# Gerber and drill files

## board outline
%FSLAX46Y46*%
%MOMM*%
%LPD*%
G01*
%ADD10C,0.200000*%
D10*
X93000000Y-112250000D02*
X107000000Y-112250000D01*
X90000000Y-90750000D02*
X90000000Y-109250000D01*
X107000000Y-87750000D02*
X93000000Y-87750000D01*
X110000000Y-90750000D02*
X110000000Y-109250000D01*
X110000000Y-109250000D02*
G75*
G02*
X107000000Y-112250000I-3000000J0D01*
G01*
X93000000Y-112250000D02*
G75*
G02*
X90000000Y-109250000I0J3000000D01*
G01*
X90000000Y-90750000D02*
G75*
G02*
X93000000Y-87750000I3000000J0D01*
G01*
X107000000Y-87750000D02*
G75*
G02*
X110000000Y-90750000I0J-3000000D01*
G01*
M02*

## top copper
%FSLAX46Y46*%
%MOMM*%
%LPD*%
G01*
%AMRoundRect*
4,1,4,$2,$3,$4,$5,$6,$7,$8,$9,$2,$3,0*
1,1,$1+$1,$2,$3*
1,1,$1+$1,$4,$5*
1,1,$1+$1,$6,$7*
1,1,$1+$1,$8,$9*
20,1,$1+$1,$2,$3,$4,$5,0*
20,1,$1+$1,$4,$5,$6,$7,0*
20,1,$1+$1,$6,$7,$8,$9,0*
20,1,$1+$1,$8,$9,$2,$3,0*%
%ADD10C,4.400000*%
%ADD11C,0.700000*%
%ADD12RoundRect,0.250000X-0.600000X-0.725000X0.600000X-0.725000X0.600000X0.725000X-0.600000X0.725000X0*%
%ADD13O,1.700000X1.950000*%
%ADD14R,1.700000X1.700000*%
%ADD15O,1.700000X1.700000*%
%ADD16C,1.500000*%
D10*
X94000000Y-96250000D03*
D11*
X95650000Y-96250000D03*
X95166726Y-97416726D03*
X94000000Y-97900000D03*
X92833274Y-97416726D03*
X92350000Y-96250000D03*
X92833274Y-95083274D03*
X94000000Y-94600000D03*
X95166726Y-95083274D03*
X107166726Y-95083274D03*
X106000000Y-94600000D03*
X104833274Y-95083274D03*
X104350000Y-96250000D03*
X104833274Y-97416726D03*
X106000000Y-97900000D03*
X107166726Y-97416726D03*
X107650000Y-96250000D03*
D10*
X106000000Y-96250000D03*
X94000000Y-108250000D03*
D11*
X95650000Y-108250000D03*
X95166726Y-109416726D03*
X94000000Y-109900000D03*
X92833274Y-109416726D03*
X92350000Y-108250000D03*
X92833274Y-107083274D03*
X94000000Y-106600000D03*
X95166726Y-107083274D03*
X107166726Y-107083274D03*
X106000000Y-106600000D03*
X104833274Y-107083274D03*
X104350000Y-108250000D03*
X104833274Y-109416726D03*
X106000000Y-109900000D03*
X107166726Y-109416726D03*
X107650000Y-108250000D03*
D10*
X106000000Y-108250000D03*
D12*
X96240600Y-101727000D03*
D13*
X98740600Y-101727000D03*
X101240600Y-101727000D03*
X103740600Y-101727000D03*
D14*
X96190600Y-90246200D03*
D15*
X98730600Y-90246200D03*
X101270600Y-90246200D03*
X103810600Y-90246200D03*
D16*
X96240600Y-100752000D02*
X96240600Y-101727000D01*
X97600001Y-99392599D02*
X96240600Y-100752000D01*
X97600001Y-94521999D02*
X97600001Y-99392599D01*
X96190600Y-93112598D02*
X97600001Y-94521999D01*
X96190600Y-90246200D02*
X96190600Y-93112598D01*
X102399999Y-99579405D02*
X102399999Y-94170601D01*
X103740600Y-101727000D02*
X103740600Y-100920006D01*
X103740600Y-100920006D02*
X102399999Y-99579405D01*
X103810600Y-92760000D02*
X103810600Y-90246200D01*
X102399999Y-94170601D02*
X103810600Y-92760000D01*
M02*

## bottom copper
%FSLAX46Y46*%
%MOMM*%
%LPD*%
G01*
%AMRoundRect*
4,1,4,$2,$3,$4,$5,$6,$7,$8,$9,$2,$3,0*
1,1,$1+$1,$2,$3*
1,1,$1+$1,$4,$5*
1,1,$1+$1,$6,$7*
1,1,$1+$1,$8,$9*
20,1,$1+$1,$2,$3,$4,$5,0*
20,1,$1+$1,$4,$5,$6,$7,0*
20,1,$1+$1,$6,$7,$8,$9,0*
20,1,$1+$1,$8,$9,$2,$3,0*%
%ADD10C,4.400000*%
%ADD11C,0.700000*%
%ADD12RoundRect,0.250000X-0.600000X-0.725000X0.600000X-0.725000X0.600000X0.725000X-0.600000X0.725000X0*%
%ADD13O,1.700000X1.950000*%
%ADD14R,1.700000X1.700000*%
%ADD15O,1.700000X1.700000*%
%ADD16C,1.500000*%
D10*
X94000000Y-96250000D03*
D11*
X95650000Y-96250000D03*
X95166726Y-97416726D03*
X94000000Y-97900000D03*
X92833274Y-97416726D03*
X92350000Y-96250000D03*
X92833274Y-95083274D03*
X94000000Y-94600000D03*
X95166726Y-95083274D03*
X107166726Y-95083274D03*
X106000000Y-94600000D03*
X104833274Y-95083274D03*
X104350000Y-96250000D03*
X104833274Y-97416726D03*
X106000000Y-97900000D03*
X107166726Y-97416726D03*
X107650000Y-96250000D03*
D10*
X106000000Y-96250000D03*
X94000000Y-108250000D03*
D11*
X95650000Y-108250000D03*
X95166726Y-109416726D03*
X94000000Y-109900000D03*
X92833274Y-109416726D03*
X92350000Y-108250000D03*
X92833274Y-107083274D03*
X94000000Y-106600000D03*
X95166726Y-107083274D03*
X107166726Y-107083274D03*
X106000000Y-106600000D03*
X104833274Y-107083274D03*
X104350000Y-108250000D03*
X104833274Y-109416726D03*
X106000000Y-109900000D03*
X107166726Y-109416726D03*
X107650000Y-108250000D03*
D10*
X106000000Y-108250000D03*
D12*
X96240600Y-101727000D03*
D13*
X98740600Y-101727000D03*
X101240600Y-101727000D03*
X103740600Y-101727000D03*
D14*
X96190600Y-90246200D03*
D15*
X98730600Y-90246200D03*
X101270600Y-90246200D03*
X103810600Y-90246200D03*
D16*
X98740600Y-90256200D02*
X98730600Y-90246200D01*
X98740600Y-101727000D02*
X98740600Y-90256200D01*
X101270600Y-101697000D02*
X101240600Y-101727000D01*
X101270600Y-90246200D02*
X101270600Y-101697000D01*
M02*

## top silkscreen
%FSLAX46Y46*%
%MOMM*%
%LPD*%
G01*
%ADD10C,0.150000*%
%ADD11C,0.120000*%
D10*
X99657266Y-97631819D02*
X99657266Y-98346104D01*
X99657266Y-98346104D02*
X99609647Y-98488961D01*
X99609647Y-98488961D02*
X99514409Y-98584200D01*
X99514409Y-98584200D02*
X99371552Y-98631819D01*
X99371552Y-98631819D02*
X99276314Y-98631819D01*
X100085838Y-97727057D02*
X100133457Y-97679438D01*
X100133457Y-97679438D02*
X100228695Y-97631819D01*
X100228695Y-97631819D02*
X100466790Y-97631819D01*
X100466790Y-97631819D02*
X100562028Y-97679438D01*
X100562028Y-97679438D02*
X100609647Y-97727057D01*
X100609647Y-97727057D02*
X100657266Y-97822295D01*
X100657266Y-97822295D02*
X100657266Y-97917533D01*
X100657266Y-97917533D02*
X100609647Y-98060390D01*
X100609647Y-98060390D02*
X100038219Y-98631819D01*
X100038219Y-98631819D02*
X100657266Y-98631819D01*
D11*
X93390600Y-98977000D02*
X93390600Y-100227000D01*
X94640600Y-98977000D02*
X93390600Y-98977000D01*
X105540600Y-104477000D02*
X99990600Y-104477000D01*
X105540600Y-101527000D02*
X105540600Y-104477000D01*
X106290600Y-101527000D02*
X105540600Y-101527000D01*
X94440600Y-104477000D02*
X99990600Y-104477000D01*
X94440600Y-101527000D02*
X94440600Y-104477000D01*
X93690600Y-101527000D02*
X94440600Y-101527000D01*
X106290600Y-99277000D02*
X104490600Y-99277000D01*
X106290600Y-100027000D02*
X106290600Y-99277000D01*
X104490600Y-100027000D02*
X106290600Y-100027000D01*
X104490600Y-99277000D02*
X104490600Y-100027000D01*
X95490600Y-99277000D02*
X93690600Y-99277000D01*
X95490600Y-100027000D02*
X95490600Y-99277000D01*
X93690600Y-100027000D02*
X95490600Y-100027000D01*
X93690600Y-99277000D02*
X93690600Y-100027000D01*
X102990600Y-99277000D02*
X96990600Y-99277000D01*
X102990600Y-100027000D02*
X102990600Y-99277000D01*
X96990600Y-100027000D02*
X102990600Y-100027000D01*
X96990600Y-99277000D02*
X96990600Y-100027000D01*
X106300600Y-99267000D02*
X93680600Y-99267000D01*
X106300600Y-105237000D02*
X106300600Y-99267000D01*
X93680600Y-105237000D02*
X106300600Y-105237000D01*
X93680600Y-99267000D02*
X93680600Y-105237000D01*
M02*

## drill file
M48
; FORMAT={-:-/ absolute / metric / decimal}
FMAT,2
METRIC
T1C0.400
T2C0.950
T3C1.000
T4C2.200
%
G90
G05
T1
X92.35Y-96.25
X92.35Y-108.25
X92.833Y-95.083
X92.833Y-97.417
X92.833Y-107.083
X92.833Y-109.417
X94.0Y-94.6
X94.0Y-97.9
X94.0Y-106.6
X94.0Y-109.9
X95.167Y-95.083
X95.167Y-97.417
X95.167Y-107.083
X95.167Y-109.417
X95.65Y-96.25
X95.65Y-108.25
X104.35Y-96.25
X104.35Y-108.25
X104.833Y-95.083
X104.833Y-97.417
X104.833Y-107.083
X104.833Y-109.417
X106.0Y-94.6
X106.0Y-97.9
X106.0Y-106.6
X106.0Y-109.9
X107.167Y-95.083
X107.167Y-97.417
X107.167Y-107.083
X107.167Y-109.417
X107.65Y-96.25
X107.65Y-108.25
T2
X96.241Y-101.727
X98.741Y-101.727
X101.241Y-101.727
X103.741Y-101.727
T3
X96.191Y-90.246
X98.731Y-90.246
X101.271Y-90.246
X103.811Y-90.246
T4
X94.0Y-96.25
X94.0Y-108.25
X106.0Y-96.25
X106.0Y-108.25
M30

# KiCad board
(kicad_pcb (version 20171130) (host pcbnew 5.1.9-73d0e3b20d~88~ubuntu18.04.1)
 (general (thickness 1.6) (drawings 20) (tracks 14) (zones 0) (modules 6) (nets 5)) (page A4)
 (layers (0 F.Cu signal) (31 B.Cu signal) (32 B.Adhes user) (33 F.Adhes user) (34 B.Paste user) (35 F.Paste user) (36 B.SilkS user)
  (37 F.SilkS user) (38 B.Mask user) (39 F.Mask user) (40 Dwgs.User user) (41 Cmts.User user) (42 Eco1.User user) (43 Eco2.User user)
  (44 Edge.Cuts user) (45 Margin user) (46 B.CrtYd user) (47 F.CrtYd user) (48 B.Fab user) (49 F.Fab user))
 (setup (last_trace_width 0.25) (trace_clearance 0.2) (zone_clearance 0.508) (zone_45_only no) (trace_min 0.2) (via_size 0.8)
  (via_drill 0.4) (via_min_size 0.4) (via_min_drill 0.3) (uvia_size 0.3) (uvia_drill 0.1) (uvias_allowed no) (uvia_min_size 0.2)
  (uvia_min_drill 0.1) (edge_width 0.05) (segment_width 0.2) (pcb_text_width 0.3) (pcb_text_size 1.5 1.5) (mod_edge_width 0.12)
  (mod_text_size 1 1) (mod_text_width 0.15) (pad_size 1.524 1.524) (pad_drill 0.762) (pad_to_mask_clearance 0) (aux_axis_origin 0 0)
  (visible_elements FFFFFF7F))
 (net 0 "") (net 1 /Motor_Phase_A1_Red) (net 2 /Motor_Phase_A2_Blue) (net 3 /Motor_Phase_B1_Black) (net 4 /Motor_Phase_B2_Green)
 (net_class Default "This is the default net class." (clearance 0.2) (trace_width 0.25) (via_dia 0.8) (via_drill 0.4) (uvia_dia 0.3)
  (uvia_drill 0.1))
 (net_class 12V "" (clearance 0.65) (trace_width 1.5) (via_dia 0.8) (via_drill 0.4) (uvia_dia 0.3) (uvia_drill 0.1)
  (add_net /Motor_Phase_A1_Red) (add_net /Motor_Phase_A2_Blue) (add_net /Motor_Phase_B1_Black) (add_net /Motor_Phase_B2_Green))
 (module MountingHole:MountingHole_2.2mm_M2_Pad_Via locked (layer F.Cu) (at 94 96.25)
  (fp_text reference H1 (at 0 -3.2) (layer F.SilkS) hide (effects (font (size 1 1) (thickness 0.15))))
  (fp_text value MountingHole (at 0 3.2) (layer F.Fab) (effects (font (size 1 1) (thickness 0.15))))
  (pad 1 thru_hole circle (at 0 0) (size 4.4 4.4) (drill 2.2) (layers *.Cu *.Mask))
  (pad 1 thru_hole circle (at 1.65 0) (size 0.7 0.7) (drill 0.4) (layers *.Cu *.Mask))
  (pad 1 thru_hole circle (at 1.166726 1.166726) (size 0.7 0.7) (drill 0.4) (layers *.Cu *.Mask))
  (pad 1 thru_hole circle (at 0 1.65) (size 0.7 0.7) (drill 0.4) (layers *.Cu *.Mask))
  (pad 1 thru_hole circle (at -1.166726 1.166726) (size 0.7 0.7) (drill 0.4) (layers *.Cu *.Mask))
  (pad 1 thru_hole circle (at -1.65 0) (size 0.7 0.7) (drill 0.4) (layers *.Cu *.Mask))
  (pad 1 thru_hole circle (at -1.166726 -1.166726) (size 0.7 0.7) (drill 0.4) (layers *.Cu *.Mask))
  (pad 1 thru_hole circle (at 0 -1.65) (size 0.7 0.7) (drill 0.4) (layers *.Cu *.Mask))
  (pad 1 thru_hole circle (at 1.166726 -1.166726) (size 0.7 0.7) (drill 0.4) (layers *.Cu *.Mask)))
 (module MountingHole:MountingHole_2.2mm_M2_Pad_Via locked (layer F.Cu) (at 106 96.25)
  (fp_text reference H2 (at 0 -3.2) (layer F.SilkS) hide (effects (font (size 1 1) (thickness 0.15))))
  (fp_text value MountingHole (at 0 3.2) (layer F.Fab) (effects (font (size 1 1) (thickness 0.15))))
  (pad 1 thru_hole circle (at 1.166726 -1.166726) (size 0.7 0.7) (drill 0.4) (layers *.Cu *.Mask))
  (pad 1 thru_hole circle (at 0 -1.65) (size 0.7 0.7) (drill 0.4) (layers *.Cu *.Mask))
  (pad 1 thru_hole circle (at -1.166726 -1.166726) (size 0.7 0.7) (drill 0.4) (layers *.Cu *.Mask))
  (pad 1 thru_hole circle (at -1.65 0) (size 0.7 0.7) (drill 0.4) (layers *.Cu *.Mask))
  (pad 1 thru_hole circle (at -1.166726 1.166726) (size 0.7 0.7) (drill 0.4) (layers *.Cu *.Mask))
  (pad 1 thru_hole circle (at 0 1.65) (size 0.7 0.7) (drill 0.4) (layers *.Cu *.Mask))
  (pad 1 thru_hole circle (at 1.166726 1.166726) (size 0.7 0.7) (drill 0.4) (layers *.Cu *.Mask))
  (pad 1 thru_hole circle (at 1.65 0) (size 0.7 0.7) (drill 0.4) (layers *.Cu *.Mask))
  (pad 1 thru_hole circle (at 0 0) (size 4.4 4.4) (drill 2.2) (layers *.Cu *.Mask)))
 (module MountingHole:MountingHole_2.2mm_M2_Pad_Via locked (layer F.Cu) (at 94 108.25)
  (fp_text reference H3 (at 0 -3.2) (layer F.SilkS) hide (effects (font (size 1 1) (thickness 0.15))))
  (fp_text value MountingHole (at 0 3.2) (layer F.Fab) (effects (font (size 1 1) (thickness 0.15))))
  (pad 1 thru_hole circle (at 0 0) (size 4.4 4.4) (drill 2.2) (layers *.Cu *.Mask))
  (pad 1 thru_hole circle (at 1.65 0) (size 0.7 0.7) (drill 0.4) (layers *.Cu *.Mask))
  (pad 1 thru_hole circle (at 1.166726 1.166726) (size 0.7 0.7) (drill 0.4) (layers *.Cu *.Mask))
  (pad 1 thru_hole circle (at 0 1.65) (size 0.7 0.7) (drill 0.4) (layers *.Cu *.Mask))
  (pad 1 thru_hole circle (at -1.166726 1.166726) (size 0.7 0.7) (drill 0.4) (layers *.Cu *.Mask))
  (pad 1 thru_hole circle (at -1.65 0) (size 0.7 0.7) (drill 0.4) (layers *.Cu *.Mask))
  (pad 1 thru_hole circle (at -1.166726 -1.166726) (size 0.7 0.7) (drill 0.4) (layers *.Cu *.Mask))
  (pad 1 thru_hole circle (at 0 -1.65) (size 0.7 0.7) (drill 0.4) (layers *.Cu *.Mask))
  (pad 1 thru_hole circle (at 1.166726 -1.166726) (size 0.7 0.7) (drill 0.4) (layers *.Cu *.Mask)))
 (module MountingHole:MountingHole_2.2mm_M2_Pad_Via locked (layer F.Cu) (at 106 108.25)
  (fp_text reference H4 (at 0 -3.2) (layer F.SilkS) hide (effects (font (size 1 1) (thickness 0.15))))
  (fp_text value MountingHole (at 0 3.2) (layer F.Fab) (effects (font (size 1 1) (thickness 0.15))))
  (pad 1 thru_hole circle (at 1.166726 -1.166726) (size 0.7 0.7) (drill 0.4) (layers *.Cu *.Mask))
  (pad 1 thru_hole circle (at 0 -1.65) (size 0.7 0.7) (drill 0.4) (layers *.Cu *.Mask))
  (pad 1 thru_hole circle (at -1.166726 -1.166726) (size 0.7 0.7) (drill 0.4) (layers *.Cu *.Mask))
  (pad 1 thru_hole circle (at -1.65 0) (size 0.7 0.7) (drill 0.4) (layers *.Cu *.Mask))
  (pad 1 thru_hole circle (at -1.166726 1.166726) (size 0.7 0.7) (drill 0.4) (layers *.Cu *.Mask))
  (pad 1 thru_hole circle (at 0 1.65) (size 0.7 0.7) (drill 0.4) (layers *.Cu *.Mask))
  (pad 1 thru_hole circle (at 1.166726 1.166726) (size 0.7 0.7) (drill 0.4) (layers *.Cu *.Mask))
  (pad 1 thru_hole circle (at 1.65 0) (size 0.7 0.7) (drill 0.4) (layers *.Cu *.Mask))
  (pad 1 thru_hole circle (at 0 0) (size 4.4 4.4) (drill 2.2) (layers *.Cu *.Mask)))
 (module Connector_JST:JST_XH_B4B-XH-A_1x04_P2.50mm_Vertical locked (layer F.Cu) (at 96.2406 101.727)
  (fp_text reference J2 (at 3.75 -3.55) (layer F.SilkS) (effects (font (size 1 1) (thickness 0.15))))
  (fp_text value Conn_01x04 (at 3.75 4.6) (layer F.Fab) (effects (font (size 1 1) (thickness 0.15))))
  (fp_line (start -2.85 -2.75) (end -2.85 -1.5) (layer F.SilkS) (width 0.12))
  (fp_line (start -1.6 -2.75) (end -2.85 -2.75) (layer F.SilkS) (width 0.12))
  (fp_line (start 9.3 2.75) (end 3.75 2.75) (layer F.SilkS) (width 0.12))
  (fp_line (start 9.3 -0.2) (end 9.3 2.75) (layer F.SilkS) (width 0.12))
  (fp_line (start 10.05 -0.2) (end 9.3 -0.2) (layer F.SilkS) (width 0.12))
  (fp_line (start -1.8 2.75) (end 3.75 2.75) (layer F.SilkS) (width 0.12))
  (fp_line (start -1.8 -0.2) (end -1.8 2.75) (layer F.SilkS) (width 0.12))
  (fp_line (start -2.55 -0.2) (end -1.8 -0.2) (layer F.SilkS) (width 0.12))
  (fp_line (start 10.05 -2.45) (end 8.25 -2.45) (layer F.SilkS) (width 0.12))
  (fp_line (start 10.05 -1.7) (end 10.05 -2.45) (layer F.SilkS) (width 0.12))
  (fp_line (start 8.25 -1.7) (end 10.05 -1.7) (layer F.SilkS) (width 0.12))
  (fp_line (start 8.25 -2.45) (end 8.25 -1.7) (layer F.SilkS) (width 0.12))
  (fp_line (start -0.75 -2.45) (end -2.55 -2.45) (layer F.SilkS) (width 0.12))
  (fp_line (start -0.75 -1.7) (end -0.75 -2.45) (layer F.SilkS) (width 0.12))
  (fp_line (start -2.55 -1.7) (end -0.75 -1.7) (layer F.SilkS) (width 0.12))
  (fp_line (start -2.55 -2.45) (end -2.55 -1.7) (layer F.SilkS) (width 0.12))
  (fp_line (start 6.75 -2.45) (end 0.75 -2.45) (layer F.SilkS) (width 0.12))
  (fp_line (start 6.75 -1.7) (end 6.75 -2.45) (layer F.SilkS) (width 0.12))
  (fp_line (start 0.75 -1.7) (end 6.75 -1.7) (layer F.SilkS) (width 0.12))
  (fp_line (start 0.75 -2.45) (end 0.75 -1.7) (layer F.SilkS) (width 0.12))
  (fp_line (start 10.06 -2.46) (end -2.56 -2.46) (layer F.SilkS) (width 0.12))
  (fp_line (start 10.06 3.51) (end 10.06 -2.46) (layer F.SilkS) (width 0.12))
  (fp_line (start -2.56 3.51) (end 10.06 3.51) (layer F.SilkS) (width 0.12))
  (fp_line (start -2.56 -2.46) (end -2.56 3.51) (layer F.SilkS) (width 0.12))
  (pad 1 thru_hole roundrect (at 0 0) (size 1.7 1.95) (drill 0.95) (layers *.Cu *.Mask) (roundrect_rratio 0.1470588235294118)
   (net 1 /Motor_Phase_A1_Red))
  (pad 2 thru_hole oval (at 2.5 0) (size 1.7 1.95) (drill 0.95) (layers *.Cu *.Mask) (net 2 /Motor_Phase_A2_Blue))
  (pad 3 thru_hole oval (at 5 0) (size 1.7 1.95) (drill 0.95) (layers *.Cu *.Mask) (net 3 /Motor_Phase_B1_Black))
  (pad 4 thru_hole oval (at 7.5 0) (size 1.7 1.95) (drill 0.95) (layers *.Cu *.Mask) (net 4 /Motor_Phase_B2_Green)))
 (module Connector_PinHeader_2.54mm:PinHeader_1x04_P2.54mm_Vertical (layer B.Cu) (at 96.1906 90.2462 270)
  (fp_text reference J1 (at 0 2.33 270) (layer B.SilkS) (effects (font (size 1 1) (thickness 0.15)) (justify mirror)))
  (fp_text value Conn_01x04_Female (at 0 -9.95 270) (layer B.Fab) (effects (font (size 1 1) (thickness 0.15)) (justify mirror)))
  (pad 1 thru_hole rect (at 0 0 270) (size 1.7 1.7) (drill 1) (layers *.Cu *.Mask) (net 1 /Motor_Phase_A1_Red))
  (pad 2 thru_hole oval (at 0 -2.54 270) (size 1.7 1.7) (drill 1) (layers *.Cu *.Mask) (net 2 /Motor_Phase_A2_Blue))
  (pad 3 thru_hole oval (at 0 -5.08 270) (size 1.7 1.7) (drill 1) (layers *.Cu *.Mask) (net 3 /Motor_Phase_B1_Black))
  (pad 4 thru_hole oval (at 0 -7.62 270) (size 1.7 1.7) (drill 1) (layers *.Cu *.Mask) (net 4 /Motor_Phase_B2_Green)))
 (gr_line (start 93 112.25) (end 107 112.25) (layer Edge.Cuts) (width 0.2))
 (gr_line (start 90 90.75) (end 90 109.25) (layer Edge.Cuts) (width 0.2))
 (gr_line (start 107 87.75) (end 93 87.75) (layer Edge.Cuts) (width 0.2))
 (gr_line (start 110 90.75) (end 110 109.25) (layer Edge.Cuts) (width 0.2))
 (gr_arc (start 107 109.25) (end 107 112.25) (angle -90) (layer Edge.Cuts) (width 0.2))
 (gr_arc (start 93 109.25) (end 90 109.25) (angle -90) (layer Edge.Cuts) (width 0.2))
 (gr_arc (start 93 90.75) (end 93 87.75) (angle -90) (layer Edge.Cuts) (width 0.2))
 (gr_arc (start 107 90.75) (end 110 90.75) (angle -90) (layer Edge.Cuts) (width 0.2))
 (segment (start 96.2406 100.752) (end 96.2406 101.727) (width 1.5) (layer F.Cu) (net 1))
 (segment (start 97.600001 99.392599) (end 96.2406 100.752) (width 1.5) (layer F.Cu) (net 1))
 (segment (start 97.600001 94.521999) (end 97.600001 99.392599) (width 1.5) (layer F.Cu) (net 1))
 (segment (start 96.1906 93.112598) (end 97.600001 94.521999) (width 1.5) (layer F.Cu) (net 1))
 (segment (start 96.1906 90.2462) (end 96.1906 93.112598) (width 1.5) (layer F.Cu) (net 1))
 (segment (start 98.7406 90.2562) (end 98.7306 90.2462) (width 1.5) (layer B.Cu) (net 2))
 (segment (start 98.7406 101.727) (end 98.7406 90.2562) (width 1.5) (layer B.Cu) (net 2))
 (segment (start 101.2706 101.697) (end 101.2406 101.727) (width 1.5) (layer B.Cu) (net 3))
 (segment (start 101.2706 90.2462) (end 101.2706 101.697) (width 1.5) (layer B.Cu) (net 3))
 (segment (start 102.399999 99.579405) (end 102.399999 94.170601) (width 1.5) (layer F.Cu) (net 4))
 (segment (start 103.7406 101.727) (end 103.7406 100.920006) (width 1.5) (layer F.Cu) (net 4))
 (segment (start 103.7406 100.920006) (end 102.399999 99.579405) (width 1.5) (layer F.Cu) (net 4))
 (segment (start 103.8106 92.76) (end 103.8106 90.2462) (width 1.5) (layer F.Cu) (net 4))
 (segment (start 102.399999 94.170601) (end 103.8106 92.76) (width 1.5) (layer F.Cu) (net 4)))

